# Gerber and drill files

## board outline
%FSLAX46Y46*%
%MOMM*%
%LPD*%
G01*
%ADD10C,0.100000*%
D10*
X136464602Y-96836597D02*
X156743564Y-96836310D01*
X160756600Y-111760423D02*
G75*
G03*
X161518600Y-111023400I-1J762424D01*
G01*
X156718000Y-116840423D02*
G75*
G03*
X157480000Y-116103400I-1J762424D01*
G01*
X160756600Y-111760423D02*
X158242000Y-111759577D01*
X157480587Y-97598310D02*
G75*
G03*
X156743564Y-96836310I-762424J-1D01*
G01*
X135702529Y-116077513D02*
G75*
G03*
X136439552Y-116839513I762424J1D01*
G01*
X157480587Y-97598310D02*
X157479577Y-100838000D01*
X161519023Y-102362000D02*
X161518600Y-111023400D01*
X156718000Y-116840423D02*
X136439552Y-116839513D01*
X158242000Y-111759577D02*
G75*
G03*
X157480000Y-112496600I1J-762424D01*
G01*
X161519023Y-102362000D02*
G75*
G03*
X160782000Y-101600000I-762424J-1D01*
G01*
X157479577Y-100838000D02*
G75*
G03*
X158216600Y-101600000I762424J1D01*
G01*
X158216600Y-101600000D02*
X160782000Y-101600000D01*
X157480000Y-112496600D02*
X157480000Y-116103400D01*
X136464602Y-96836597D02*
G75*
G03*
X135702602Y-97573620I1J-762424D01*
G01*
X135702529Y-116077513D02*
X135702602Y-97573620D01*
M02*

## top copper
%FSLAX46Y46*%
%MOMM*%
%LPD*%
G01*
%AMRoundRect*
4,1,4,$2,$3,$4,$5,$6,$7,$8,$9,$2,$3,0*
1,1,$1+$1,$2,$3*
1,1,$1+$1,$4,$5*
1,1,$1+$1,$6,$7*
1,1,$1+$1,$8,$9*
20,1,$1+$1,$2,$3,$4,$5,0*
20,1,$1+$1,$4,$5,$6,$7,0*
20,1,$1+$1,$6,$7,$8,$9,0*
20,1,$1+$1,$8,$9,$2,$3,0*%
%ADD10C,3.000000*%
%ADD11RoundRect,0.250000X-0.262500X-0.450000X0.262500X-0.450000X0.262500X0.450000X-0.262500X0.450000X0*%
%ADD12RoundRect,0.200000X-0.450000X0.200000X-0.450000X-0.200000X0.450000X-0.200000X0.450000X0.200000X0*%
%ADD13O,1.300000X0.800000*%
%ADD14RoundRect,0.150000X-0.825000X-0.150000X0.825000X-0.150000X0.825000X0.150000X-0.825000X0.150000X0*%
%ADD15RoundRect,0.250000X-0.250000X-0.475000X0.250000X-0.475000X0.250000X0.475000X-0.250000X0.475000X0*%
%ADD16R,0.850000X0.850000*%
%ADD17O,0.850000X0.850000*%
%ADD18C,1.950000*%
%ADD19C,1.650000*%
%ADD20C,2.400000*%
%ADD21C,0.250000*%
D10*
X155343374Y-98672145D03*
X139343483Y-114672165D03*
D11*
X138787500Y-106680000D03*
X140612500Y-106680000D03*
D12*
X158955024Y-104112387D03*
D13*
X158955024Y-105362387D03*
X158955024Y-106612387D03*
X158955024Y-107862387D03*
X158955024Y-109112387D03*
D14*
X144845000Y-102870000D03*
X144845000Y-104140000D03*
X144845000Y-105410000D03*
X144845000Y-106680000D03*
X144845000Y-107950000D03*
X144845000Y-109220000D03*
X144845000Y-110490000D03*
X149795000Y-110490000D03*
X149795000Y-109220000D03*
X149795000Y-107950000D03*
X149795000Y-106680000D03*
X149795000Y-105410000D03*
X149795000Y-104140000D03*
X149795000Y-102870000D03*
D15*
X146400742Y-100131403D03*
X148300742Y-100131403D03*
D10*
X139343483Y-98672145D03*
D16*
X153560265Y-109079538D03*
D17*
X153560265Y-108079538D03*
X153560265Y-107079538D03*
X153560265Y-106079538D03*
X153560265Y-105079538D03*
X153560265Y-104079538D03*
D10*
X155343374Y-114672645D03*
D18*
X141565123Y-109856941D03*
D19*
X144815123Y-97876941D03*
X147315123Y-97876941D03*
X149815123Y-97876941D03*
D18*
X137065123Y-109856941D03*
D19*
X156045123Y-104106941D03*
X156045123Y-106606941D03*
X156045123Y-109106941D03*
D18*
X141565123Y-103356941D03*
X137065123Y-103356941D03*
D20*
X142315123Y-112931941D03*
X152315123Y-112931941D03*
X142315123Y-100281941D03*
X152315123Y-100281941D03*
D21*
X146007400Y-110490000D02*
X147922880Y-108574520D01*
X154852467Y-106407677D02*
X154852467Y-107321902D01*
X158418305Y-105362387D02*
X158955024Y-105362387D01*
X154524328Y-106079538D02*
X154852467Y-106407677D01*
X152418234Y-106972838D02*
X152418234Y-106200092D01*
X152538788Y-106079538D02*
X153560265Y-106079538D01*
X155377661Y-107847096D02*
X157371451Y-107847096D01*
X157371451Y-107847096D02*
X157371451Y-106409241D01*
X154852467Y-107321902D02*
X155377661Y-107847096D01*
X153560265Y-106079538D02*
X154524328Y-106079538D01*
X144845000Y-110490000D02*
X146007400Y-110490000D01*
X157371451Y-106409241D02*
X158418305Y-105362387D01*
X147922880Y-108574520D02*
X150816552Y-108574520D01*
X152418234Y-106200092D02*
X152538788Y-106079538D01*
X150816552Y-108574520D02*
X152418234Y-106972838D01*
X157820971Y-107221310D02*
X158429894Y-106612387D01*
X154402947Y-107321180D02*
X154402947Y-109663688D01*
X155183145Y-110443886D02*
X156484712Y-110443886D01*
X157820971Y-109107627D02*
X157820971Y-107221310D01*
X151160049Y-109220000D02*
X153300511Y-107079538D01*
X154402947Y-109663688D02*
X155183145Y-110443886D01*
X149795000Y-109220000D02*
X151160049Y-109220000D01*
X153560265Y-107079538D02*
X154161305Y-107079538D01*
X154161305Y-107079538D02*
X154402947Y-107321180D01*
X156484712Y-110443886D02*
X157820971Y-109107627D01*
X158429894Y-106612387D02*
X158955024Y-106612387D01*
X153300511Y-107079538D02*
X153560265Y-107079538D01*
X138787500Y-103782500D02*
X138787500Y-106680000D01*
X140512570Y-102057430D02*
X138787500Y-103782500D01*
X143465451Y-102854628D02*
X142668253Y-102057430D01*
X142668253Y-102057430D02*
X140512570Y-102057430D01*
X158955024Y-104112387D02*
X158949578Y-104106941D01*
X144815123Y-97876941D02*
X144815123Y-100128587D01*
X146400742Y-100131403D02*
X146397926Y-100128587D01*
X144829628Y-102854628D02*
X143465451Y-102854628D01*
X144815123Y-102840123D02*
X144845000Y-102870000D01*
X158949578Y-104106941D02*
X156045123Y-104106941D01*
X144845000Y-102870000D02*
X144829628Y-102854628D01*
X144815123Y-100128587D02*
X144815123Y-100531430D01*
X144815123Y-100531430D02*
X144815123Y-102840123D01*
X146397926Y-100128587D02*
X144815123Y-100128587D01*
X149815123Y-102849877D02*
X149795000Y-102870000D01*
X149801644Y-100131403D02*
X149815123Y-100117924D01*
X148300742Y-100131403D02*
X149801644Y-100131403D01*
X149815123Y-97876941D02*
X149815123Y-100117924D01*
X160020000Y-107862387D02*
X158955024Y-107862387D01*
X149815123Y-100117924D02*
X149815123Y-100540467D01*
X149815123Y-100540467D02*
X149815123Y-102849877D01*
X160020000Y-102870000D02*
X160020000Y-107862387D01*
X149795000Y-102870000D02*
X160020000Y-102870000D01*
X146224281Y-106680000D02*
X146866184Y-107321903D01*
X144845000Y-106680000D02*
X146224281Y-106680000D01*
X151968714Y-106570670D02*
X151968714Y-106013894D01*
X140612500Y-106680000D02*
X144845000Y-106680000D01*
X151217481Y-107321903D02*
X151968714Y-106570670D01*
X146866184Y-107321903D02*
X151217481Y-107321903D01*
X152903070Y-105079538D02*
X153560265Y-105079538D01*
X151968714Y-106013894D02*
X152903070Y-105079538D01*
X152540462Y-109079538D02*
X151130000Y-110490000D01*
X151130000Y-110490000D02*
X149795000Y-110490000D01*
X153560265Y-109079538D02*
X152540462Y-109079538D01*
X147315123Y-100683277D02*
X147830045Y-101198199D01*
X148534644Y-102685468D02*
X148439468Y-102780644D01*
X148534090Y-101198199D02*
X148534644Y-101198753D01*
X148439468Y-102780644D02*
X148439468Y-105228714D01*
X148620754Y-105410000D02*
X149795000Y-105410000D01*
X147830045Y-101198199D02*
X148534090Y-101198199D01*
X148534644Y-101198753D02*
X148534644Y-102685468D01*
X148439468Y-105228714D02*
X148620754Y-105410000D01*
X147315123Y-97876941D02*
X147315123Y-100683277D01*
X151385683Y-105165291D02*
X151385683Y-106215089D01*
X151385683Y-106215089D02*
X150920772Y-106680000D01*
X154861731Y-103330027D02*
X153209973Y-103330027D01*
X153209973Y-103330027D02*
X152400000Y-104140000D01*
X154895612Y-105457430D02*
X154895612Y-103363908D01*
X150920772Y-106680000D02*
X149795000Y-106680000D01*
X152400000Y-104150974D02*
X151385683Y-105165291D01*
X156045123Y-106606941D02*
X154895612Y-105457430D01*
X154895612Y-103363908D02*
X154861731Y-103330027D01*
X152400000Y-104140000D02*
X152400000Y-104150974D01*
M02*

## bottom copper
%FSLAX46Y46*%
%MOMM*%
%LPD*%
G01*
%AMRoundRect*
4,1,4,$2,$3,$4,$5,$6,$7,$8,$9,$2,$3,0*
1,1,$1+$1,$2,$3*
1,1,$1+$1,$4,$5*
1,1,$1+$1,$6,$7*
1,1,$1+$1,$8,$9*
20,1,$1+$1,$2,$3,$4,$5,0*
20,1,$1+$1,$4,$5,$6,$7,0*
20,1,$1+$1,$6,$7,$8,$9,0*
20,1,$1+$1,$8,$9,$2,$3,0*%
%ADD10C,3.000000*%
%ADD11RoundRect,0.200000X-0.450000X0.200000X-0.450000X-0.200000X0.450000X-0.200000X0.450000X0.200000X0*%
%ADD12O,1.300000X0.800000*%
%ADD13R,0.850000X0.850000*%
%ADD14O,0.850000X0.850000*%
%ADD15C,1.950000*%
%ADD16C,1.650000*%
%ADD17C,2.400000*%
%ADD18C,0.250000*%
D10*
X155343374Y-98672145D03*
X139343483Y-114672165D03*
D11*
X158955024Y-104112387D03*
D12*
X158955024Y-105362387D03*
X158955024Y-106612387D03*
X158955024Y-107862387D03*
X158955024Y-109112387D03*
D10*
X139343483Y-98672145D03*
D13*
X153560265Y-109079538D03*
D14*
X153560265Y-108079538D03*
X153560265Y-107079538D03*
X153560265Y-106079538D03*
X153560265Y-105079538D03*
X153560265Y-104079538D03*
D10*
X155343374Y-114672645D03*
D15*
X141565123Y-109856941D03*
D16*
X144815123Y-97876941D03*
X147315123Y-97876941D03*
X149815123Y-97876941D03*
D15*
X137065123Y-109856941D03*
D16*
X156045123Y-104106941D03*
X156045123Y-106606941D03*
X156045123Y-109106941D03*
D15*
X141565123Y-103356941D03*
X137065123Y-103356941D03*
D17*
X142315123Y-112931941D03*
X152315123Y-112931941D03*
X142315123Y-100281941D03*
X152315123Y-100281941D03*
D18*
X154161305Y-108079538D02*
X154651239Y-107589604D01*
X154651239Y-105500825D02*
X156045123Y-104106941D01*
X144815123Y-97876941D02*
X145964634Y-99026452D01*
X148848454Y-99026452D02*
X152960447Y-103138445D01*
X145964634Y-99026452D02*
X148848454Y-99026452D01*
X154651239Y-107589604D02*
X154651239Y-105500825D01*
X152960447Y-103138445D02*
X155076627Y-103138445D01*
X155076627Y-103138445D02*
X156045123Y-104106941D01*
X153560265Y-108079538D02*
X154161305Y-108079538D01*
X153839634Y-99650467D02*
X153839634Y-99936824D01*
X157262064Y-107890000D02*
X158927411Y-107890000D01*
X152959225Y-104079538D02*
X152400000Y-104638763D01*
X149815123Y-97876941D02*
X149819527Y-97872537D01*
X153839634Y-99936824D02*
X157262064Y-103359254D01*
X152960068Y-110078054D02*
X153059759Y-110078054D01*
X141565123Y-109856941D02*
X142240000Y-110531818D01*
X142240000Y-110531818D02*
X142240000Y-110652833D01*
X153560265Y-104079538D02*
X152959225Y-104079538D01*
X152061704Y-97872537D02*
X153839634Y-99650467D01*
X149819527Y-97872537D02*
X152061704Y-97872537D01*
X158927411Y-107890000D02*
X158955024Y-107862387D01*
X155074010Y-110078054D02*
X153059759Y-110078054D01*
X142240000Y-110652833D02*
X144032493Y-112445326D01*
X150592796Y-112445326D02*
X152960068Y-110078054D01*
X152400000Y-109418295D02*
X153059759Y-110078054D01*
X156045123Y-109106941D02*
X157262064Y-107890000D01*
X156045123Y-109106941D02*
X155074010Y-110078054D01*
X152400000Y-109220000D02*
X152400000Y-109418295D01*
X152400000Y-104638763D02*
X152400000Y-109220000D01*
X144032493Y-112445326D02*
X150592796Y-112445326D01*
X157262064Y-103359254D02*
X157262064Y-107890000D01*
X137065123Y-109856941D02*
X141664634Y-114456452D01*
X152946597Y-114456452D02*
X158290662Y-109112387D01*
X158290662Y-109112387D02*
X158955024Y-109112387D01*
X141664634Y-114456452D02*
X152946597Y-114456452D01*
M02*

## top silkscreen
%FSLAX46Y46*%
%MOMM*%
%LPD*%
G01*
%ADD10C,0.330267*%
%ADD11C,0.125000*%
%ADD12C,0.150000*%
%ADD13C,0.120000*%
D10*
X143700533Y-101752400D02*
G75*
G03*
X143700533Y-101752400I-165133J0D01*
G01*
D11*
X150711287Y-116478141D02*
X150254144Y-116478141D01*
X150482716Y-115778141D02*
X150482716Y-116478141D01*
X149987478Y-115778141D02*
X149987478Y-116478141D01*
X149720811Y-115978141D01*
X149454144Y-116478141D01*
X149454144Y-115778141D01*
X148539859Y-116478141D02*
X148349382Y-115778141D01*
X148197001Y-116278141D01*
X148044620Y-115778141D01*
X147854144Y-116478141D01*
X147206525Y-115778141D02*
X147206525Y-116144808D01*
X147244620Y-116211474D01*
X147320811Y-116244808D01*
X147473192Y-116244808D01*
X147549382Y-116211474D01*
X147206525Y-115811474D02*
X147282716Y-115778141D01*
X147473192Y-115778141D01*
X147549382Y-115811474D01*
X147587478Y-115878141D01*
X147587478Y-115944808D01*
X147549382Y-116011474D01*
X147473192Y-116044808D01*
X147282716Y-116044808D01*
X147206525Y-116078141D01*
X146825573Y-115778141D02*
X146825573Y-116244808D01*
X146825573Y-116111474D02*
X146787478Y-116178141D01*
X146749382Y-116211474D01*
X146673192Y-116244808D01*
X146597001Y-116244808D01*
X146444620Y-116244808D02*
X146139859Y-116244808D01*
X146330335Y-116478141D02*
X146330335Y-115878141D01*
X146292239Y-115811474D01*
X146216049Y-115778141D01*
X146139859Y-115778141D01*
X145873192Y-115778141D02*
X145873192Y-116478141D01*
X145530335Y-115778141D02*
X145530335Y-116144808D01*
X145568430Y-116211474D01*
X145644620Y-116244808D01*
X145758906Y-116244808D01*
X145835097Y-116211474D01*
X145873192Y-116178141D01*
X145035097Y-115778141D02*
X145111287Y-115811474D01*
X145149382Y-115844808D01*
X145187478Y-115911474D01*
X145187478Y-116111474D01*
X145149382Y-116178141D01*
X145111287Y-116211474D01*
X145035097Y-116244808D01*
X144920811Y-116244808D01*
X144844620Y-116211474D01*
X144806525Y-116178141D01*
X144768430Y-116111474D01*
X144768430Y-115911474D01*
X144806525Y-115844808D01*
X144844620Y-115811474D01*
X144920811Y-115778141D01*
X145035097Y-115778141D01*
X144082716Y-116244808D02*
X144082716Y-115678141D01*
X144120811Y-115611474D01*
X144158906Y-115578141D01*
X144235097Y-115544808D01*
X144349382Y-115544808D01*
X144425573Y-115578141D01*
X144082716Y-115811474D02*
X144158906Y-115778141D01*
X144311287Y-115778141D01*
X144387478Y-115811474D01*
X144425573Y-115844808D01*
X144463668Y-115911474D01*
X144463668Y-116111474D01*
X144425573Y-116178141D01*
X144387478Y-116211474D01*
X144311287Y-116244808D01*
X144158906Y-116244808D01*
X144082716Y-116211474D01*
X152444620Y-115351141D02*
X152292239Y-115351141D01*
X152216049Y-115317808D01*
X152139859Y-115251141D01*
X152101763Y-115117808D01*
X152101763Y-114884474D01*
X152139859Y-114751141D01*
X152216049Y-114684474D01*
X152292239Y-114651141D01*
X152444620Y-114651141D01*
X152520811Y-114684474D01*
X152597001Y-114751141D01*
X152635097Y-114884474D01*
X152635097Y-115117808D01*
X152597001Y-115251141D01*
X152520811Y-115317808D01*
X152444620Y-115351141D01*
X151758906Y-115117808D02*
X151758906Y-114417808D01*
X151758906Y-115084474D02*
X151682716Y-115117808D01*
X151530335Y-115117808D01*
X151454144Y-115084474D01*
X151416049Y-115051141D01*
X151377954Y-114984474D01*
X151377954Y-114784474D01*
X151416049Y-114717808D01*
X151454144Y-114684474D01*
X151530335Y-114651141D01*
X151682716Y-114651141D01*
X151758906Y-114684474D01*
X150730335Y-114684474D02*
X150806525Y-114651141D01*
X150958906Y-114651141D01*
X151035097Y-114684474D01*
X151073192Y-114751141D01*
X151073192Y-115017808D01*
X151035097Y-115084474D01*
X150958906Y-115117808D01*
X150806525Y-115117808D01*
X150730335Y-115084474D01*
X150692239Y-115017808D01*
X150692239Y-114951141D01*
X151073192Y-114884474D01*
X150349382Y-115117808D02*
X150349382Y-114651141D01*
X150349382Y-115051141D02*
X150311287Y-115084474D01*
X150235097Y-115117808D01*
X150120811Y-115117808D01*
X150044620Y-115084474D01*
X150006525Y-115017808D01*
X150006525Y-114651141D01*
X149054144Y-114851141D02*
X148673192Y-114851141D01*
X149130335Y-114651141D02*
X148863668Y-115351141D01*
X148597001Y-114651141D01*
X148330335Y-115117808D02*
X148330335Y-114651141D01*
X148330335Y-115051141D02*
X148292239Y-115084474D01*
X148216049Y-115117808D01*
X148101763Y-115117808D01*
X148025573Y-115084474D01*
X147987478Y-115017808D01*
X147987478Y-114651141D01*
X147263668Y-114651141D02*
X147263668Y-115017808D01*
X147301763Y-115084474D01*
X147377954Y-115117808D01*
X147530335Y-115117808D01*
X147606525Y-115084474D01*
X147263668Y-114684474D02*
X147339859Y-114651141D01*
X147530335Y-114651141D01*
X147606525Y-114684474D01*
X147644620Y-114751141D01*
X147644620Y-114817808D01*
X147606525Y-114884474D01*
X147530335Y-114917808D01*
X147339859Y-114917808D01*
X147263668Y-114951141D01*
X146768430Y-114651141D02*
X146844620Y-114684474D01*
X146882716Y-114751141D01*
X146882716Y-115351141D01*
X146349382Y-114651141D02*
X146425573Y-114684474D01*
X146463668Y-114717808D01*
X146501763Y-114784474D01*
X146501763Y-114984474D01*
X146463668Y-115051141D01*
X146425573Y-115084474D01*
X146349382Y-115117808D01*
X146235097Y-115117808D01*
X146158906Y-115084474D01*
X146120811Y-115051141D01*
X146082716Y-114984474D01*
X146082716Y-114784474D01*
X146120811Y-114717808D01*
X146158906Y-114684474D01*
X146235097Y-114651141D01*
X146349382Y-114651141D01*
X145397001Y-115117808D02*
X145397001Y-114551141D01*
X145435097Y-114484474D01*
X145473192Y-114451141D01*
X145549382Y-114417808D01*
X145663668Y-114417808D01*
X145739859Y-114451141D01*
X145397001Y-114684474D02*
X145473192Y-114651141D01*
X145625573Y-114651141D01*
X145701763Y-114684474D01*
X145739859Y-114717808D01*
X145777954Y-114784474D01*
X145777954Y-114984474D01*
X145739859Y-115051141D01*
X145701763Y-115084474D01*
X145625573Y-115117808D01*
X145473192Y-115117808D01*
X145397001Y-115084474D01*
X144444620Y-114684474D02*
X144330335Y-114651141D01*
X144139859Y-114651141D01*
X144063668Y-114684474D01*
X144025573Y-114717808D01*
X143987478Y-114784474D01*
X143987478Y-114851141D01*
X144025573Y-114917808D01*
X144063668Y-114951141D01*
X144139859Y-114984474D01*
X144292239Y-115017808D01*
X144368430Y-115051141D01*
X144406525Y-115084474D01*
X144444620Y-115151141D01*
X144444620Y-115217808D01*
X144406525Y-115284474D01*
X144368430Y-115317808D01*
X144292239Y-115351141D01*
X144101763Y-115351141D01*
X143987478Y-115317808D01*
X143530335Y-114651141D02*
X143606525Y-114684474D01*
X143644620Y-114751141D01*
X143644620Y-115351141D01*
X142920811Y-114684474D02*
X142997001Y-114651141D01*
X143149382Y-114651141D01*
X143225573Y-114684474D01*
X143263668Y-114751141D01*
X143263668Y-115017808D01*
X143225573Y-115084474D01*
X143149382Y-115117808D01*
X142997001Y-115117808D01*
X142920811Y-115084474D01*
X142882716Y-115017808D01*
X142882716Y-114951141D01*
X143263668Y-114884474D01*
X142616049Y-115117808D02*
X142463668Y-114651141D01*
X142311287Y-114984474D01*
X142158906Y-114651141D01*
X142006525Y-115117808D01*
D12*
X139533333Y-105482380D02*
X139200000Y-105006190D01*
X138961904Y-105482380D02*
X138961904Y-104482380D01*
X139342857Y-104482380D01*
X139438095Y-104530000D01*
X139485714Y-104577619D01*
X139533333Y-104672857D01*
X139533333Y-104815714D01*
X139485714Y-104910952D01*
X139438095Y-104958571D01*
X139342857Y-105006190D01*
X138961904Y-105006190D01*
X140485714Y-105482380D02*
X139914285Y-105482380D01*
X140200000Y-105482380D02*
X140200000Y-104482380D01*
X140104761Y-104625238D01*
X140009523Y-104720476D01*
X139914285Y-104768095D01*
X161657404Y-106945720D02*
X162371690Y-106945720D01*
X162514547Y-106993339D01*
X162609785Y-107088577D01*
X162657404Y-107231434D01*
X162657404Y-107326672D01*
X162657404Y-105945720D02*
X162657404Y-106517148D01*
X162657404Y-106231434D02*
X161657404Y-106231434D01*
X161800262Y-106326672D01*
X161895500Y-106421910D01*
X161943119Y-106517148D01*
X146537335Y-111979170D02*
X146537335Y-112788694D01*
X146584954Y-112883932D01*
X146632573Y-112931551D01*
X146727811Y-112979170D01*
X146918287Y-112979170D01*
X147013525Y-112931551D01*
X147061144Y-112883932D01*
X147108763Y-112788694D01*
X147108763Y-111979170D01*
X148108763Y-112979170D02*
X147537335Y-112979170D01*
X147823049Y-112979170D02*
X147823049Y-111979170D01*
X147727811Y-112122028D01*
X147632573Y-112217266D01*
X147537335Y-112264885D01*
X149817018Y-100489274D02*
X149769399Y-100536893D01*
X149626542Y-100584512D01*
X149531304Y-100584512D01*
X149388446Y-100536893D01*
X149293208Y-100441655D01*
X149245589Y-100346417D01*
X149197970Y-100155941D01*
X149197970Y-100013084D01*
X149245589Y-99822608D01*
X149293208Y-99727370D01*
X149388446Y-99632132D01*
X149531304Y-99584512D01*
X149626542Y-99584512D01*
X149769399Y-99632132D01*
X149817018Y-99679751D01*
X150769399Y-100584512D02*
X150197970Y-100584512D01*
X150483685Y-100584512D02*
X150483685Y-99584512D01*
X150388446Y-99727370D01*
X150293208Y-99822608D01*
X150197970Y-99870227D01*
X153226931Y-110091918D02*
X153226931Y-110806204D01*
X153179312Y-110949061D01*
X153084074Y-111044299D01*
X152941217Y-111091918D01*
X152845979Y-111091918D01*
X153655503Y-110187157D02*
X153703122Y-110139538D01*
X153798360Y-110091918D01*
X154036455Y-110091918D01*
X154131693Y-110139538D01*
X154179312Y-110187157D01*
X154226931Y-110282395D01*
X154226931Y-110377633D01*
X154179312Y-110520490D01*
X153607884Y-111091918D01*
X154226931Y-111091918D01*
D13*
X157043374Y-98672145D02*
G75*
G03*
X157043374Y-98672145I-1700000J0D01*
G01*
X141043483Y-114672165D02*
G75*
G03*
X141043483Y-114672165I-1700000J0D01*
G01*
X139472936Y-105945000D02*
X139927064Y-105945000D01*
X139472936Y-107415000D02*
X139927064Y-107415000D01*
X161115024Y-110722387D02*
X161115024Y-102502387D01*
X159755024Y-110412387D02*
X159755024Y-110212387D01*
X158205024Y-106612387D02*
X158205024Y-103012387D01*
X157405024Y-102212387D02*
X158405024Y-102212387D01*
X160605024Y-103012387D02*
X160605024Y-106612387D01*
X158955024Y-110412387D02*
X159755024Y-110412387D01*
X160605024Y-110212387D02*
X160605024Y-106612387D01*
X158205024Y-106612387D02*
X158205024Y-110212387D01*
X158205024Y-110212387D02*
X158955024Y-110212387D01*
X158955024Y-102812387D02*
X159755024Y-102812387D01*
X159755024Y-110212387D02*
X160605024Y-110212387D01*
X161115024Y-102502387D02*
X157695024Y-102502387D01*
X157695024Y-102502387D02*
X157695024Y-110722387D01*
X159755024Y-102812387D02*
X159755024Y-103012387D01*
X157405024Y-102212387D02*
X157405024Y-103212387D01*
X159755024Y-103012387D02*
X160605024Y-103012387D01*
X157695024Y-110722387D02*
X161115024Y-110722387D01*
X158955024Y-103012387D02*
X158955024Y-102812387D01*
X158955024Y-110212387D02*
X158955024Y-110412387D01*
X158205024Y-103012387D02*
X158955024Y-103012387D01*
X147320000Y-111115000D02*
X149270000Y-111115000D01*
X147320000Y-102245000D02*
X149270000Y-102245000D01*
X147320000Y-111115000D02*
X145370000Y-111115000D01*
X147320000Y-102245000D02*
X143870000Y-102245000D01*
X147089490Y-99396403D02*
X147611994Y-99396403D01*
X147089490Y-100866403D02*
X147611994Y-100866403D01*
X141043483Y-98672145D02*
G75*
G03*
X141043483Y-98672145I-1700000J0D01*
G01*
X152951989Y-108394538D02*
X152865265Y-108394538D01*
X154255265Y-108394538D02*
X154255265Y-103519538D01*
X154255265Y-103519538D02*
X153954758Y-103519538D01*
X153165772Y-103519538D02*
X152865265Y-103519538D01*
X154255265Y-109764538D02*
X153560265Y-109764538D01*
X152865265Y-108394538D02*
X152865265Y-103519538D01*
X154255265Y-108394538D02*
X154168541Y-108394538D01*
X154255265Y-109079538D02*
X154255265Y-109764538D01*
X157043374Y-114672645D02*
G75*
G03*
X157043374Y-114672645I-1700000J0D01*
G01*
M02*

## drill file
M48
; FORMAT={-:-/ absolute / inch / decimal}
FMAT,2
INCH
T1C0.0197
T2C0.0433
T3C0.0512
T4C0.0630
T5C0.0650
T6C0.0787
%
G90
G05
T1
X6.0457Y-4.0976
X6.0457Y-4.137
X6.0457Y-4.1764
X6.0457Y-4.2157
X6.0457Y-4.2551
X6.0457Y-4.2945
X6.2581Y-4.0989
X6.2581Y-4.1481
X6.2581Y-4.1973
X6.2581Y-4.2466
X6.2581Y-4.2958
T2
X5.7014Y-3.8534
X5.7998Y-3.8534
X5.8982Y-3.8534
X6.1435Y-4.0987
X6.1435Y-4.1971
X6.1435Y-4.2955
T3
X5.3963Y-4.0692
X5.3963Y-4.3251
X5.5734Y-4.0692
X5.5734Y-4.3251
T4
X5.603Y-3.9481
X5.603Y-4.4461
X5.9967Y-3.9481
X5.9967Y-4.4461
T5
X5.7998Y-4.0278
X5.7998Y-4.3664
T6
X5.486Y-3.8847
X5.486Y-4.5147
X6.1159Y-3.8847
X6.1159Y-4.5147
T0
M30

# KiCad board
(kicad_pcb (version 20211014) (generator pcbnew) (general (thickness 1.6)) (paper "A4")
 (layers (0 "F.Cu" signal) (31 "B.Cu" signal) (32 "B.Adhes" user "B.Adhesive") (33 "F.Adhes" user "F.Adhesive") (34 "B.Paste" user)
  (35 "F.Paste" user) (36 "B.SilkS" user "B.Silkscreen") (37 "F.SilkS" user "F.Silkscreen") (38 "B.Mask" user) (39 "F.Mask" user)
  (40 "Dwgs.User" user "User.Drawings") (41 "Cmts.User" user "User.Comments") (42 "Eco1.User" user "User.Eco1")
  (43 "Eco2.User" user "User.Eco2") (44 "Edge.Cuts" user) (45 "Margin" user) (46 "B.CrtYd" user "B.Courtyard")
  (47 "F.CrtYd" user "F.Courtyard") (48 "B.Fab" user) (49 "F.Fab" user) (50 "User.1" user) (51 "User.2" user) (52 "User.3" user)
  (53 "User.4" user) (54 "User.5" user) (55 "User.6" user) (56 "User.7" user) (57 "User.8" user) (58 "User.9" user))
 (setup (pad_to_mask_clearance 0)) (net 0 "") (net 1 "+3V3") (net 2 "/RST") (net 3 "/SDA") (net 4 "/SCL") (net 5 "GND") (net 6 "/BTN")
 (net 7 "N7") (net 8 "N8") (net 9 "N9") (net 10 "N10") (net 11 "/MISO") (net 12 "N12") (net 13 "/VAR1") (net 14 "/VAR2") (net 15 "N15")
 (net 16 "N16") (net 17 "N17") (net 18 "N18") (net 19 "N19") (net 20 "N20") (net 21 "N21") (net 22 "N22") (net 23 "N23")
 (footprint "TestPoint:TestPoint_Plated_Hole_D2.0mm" (layer "F.Cu") (at 155.343374 98.672145) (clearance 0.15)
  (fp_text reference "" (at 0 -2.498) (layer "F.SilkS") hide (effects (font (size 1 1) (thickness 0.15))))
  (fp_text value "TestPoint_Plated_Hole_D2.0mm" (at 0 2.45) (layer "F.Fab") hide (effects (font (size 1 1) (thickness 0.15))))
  (fp_circle (center 0 0) (end 0 -1.7) (layer "F.SilkS") (width 0.12) (fill none))
  (pad "" thru_hole circle locked (at 0 0) (size 3 3) (drill 2) (layers *.Cu *.Mask)))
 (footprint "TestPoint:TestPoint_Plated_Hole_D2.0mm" (layer "F.Cu") (at 139.343483 114.672165) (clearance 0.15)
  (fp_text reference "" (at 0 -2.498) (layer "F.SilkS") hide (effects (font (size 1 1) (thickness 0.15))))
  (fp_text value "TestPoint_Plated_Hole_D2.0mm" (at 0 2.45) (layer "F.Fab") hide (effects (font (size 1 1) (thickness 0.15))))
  (fp_circle (center 0 0) (end 0 -1.7) (layer "F.SilkS") (width 0.12) (fill none))
  (pad "" thru_hole circle locked (at 0 0) (size 3 3) (drill 2) (layers *.Cu *.Mask)))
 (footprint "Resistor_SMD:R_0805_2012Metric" (layer "F.Cu") (at 139.7 106.68)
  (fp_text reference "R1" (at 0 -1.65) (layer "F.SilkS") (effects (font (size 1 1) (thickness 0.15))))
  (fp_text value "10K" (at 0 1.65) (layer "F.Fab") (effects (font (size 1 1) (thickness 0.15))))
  (fp_line (start -0.227064 -0.735) (end 0.227064 -0.735) (layer "F.SilkS") (width 0.12))
  (fp_line (start -0.227064 0.735) (end 0.227064 0.735) (layer "F.SilkS") (width 0.12))
  (pad "1" smd roundrect locked (at -0.9125 0) (size 1.025 1.4) (layers "F.Cu" "F.Paste" "F.Mask") (roundrect_rratio 0.243902439)
   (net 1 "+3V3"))
  (pad "2" smd roundrect locked (at 0.9125 0) (size 1.025 1.4) (layers "F.Cu" "F.Paste" "F.Mask") (roundrect_rratio 0.243902439)
   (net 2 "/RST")))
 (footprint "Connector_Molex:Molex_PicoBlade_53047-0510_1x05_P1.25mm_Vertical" (layer "F.Cu") (at 158.955024 104.112387 -90)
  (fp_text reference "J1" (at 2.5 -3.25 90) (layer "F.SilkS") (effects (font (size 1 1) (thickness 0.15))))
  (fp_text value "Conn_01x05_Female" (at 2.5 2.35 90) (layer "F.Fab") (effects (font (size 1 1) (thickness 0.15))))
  (fp_line (start 6.61 -2.16) (end -1.61 -2.16) (layer "F.SilkS") (width 0.12))
  (fp_line (start 6.3 -0.8) (end 6.1 -0.8) (layer "F.SilkS") (width 0.12))
  (fp_line (start 2.5 0.75) (end -1.1 0.75) (layer "F.SilkS") (width 0.12))
  (fp_line (start -1.9 1.55) (end -1.9 0.55) (layer "F.SilkS") (width 0.12))
  (fp_line (start -1.1 -1.65) (end 2.5 -1.65) (layer "F.SilkS") (width 0.12))
  (fp_line (start 6.3 0) (end 6.3 -0.8) (layer "F.SilkS") (width 0.12))
  (fp_line (start 6.1 -1.65) (end 2.5 -1.65) (layer "F.SilkS") (width 0.12))
  (fp_line (start 2.5 0.75) (end 6.1 0.75) (layer "F.SilkS") (width 0.12))
  (fp_line (start 6.1 0.75) (end 6.1 0) (layer "F.SilkS") (width 0.12))
  (fp_line (start -1.3 0) (end -1.3 -0.8) (layer "F.SilkS") (width 0.12))
  (fp_line (start 6.1 -0.8) (end 6.1 -1.65) (layer "F.SilkS") (width 0.12))
  (fp_line (start -1.61 -2.16) (end -1.61 1.26) (layer "F.SilkS") (width 0.12))
  (fp_line (start -1.61 1.26) (end 6.61 1.26) (layer "F.SilkS") (width 0.12))
  (fp_line (start -1.3 -0.8) (end -1.1 -0.8) (layer "F.SilkS") (width 0.12))
  (fp_line (start -1.9 1.55) (end -0.9 1.55) (layer "F.SilkS") (width 0.12))
  (fp_line (start -1.1 -0.8) (end -1.1 -1.65) (layer "F.SilkS") (width 0.12))
  (fp_line (start 6.61 1.26) (end 6.61 -2.16) (layer "F.SilkS") (width 0.12))
  (fp_line (start -1.1 0) (end -1.3 0) (layer "F.SilkS") (width 0.12))
  (fp_line (start 6.1 0) (end 6.3 0) (layer "F.SilkS") (width 0.12))
  (fp_line (start -1.1 0.75) (end -1.1 0) (layer "F.SilkS") (width 0.12))
  (pad "1" thru_hole roundrect locked (at 0 0 270) (size 0.8 1.3) (drill 0.5) (layers *.Cu *.Mask) (roundrect_rratio 0.25) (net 1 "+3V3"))
  (pad "2" thru_hole oval locked (at 1.25 0 270) (size 0.8 1.3) (drill 0.5) (layers *.Cu *.Mask) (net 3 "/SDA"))
  (pad "3" thru_hole oval locked (at 2.5 0 270) (size 0.8 1.3) (drill 0.5) (layers *.Cu *.Mask) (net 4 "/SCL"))
  (pad "4" thru_hole oval locked (at 3.75 0 270) (size 0.8 1.3) (drill 0.5) (layers *.Cu *.Mask) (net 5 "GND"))
  (pad "5" thru_hole oval locked (at 5 0 270) (size 0.8 1.3) (drill 0.5) (layers *.Cu *.Mask) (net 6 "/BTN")))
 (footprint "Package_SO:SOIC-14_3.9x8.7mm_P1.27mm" (layer "F.Cu") (at 147.32 106.68) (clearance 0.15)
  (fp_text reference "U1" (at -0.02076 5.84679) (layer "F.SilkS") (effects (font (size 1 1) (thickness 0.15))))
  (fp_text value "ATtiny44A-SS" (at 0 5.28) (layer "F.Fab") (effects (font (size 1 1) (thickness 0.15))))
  (fp_line (start 0 4.435) (end 1.95 4.435) (layer "F.SilkS") (width 0.12))
  (fp_line (start 0 -4.435) (end 1.95 -4.435) (layer "F.SilkS") (width 0.12))
  (fp_line (start 0 4.435) (end -1.95 4.435) (layer "F.SilkS") (width 0.12))
  (fp_line (start 0 -4.435) (end -3.45 -4.435) (layer "F.SilkS") (width 0.12))
  (pad "1" smd roundrect locked (at -2.475 -3.81) (size 1.95 0.6) (layers "F.Cu" "F.Paste" "F.Mask") (roundrect_rratio 0.25) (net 1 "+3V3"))
  (pad "2" smd roundrect locked (at -2.475 -2.54) (size 1.95 0.6) (layers "F.Cu" "F.Paste" "F.Mask") (roundrect_rratio 0.25) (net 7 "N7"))
  (pad "3" smd roundrect locked (at -2.475 -1.27) (size 1.95 0.6) (layers "F.Cu" "F.Paste" "F.Mask") (roundrect_rratio 0.25) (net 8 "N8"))
  (pad "4" smd roundrect locked (at -2.475 0) (size 1.95 0.6) (layers "F.Cu" "F.Paste" "F.Mask") (roundrect_rratio 0.25) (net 2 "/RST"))
  (pad "5" smd roundrect locked (at -2.475 1.27) (size 1.95 0.6) (layers "F.Cu" "F.Paste" "F.Mask") (roundrect_rratio 0.25) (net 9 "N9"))
  (pad "6" smd roundrect locked (at -2.475 2.54) (size 1.95 0.6) (layers "F.Cu" "F.Paste" "F.Mask") (roundrect_rratio 0.25) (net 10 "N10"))
  (pad "7" smd roundrect locked (at -2.475 3.81) (size 1.95 0.6) (layers "F.Cu" "F.Paste" "F.Mask") (roundrect_rratio 0.25) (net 3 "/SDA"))
  (pad "8" smd roundrect locked (at 2.475 3.81) (size 1.95 0.6) (layers "F.Cu" "F.Paste" "F.Mask") (roundrect_rratio 0.25) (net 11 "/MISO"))
  (pad "9" smd roundrect locked (at 2.475 2.54) (size 1.95 0.6) (layers "F.Cu" "F.Paste" "F.Mask") (roundrect_rratio 0.25) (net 4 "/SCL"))
  (pad "10" smd roundrect locked (at 2.475 1.27) (size 1.95 0.6) (layers "F.Cu" "F.Paste" "F.Mask") (roundrect_rratio 0.25) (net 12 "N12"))
  (pad "11" smd roundrect locked (at 2.475 0) (size 1.95 0.6) (layers "F.Cu" "F.Paste" "F.Mask") (roundrect_rratio 0.25) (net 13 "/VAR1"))
  (pad "12" smd roundrect locked (at 2.475 -1.27) (size 1.95 0.6) (layers "F.Cu" "F.Paste" "F.Mask") (roundrect_rratio 0.25)
   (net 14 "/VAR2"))
  (pad "13" smd roundrect locked (at 2.475 -2.54) (size 1.95 0.6) (layers "F.Cu" "F.Paste" "F.Mask") (roundrect_rratio 0.25) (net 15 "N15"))
  (pad "14" smd roundrect locked (at 2.475 -3.81) (size 1.95 0.6) (layers "F.Cu" "F.Paste" "F.Mask") (roundrect_rratio 0.25) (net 5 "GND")))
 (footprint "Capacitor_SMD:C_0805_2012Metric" (layer "F.Cu") (at 147.350742 100.131403)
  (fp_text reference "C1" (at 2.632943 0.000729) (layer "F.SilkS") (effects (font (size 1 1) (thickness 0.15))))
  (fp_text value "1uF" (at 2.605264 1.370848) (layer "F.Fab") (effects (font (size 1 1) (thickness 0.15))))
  (fp_line (start -0.261252 -0.735) (end 0.261252 -0.735) (layer "F.SilkS") (width 0.12))
  (fp_line (start -0.261252 0.735) (end 0.261252 0.735) (layer "F.SilkS") (width 0.12))
  (pad "1" smd roundrect locked (at -0.95 0) (size 1 1.45) (layers "F.Cu" "F.Paste" "F.Mask") (roundrect_rratio 0.25) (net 1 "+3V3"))
  (pad "2" smd roundrect locked (at 0.95 0) (size 1 1.45) (layers "F.Cu" "F.Paste" "F.Mask") (roundrect_rratio 0.25) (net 5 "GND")))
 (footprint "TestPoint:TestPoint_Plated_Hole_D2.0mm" (layer "F.Cu") (at 139.343483 98.672145)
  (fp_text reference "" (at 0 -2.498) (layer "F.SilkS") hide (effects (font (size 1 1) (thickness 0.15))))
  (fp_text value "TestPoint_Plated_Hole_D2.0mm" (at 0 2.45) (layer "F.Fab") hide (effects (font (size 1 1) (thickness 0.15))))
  (fp_circle (center 0 0) (end 0 -1.7) (layer "F.SilkS") (width 0.12) (fill none))
  (pad "" thru_hole circle locked (at 0 0) (size 3 3) (drill 2) (layers *.Cu *.Mask)))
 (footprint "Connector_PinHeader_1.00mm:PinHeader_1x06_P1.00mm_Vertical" (layer "F.Cu") (at 153.560265 109.079538 180) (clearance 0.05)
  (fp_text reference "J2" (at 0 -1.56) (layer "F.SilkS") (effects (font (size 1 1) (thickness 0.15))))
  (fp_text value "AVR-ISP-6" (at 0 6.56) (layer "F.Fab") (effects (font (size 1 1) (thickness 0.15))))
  (fp_line (start 0.608276 0.685) (end 0.695 0.685) (layer "F.SilkS") (width 0.12))
  (fp_line (start -0.695 0.685) (end -0.695 5.56) (layer "F.SilkS") (width 0.12))
  (fp_line (start -0.695 5.56) (end -0.394493 5.56) (layer "F.SilkS") (width 0.12))
  (fp_line (start 0.394493 5.56) (end 0.695 5.56) (layer "F.SilkS") (width 0.12))
  (fp_line (start -0.695 -0.685) (end 0 -0.685) (layer "F.SilkS") (width 0.12))
  (fp_line (start 0.695 0.685) (end 0.695 5.56) (layer "F.SilkS") (width 0.12))
  (fp_line (start -0.695 0.685) (end -0.608276 0.685) (layer "F.SilkS") (width 0.12))
  (fp_line (start -0.695 0) (end -0.695 -0.685) (layer "F.SilkS") (width 0.12))
  (pad "1" thru_hole rect locked (at 0 0 180) (size 0.85 0.85) (drill 0.5) (layers *.Cu *.Mask) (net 11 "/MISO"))
  (pad "2" thru_hole oval locked (at 0 1 180) (size 0.85 0.85) (drill 0.5) (layers *.Cu *.Mask) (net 1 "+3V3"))
  (pad "3" thru_hole oval locked (at 0 2 180) (size 0.85 0.85) (drill 0.5) (layers *.Cu *.Mask) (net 4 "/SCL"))
  (pad "4" thru_hole oval locked (at 0 3 180) (size 0.85 0.85) (drill 0.5) (layers *.Cu *.Mask) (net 3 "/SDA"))
  (pad "5" thru_hole oval locked (at 0 4 180) (size 0.85 0.85) (drill 0.5) (layers *.Cu *.Mask) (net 2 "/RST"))
  (pad "6" thru_hole oval locked (at 0 5 180) (size 0.85 0.85) (drill 0.5) (layers *.Cu *.Mask) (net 5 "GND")))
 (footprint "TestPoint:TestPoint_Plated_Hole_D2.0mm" (layer "F.Cu") (at 155.343374 114.672645)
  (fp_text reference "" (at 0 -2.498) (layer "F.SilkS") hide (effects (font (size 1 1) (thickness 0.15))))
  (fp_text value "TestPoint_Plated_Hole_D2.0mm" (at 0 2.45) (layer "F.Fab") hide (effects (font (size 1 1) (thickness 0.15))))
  (fp_circle (center 0 0) (end 0 -1.7) (layer "F.SilkS") (width 0.12) (fill none))
  (pad "" thru_hole circle locked (at 0 0) (size 3 3) (drill 2) (layers *.Cu *.Mask)))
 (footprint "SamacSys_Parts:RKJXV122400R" (layer "B.Cu") (at 144.815123 97.876941 90)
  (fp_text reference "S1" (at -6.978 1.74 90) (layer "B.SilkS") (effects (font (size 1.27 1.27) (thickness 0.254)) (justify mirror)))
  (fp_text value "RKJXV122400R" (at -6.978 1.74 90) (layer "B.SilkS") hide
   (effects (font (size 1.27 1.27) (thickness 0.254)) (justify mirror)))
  (pad "A1" thru_hole circle locked (at -11.98 -3.25 90) (size 1.95 1.95) (drill 1.3) (layers *.Cu *.Mask) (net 5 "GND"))
  (pad "A11" thru_hole circle locked (at 0 0 90) (size 1.65 1.65) (drill 1.1) (layers *.Cu *.Mask) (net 1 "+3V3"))
  (pad "A12" thru_hole circle locked (at 0 2.5 90) (size 1.65 1.65) (drill 1.1) (layers *.Cu *.Mask) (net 14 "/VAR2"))
  (pad "A13" thru_hole circle locked (at 0 5 90) (size 1.65 1.65) (drill 1.1) (layers *.Cu *.Mask) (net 5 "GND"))
  (pad "B1" thru_hole circle locked (at -11.98 -7.75 90) (size 1.95 1.95) (drill 1.3) (layers *.Cu *.Mask) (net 6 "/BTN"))
  (pad "B11" thru_hole circle locked (at -6.23 11.23 90) (size 1.65 1.65) (drill 1.1) (layers *.Cu *.Mask) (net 1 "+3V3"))
  (pad "B12" thru_hole circle locked (at -8.73 11.23 90) (size 1.65 1.65) (drill 1.1) (layers *.Cu *.Mask) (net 13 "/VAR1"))
  (pad "B13" thru_hole circle locked (at -11.23 11.23 90) (size 1.65 1.65) (drill 1.1) (layers *.Cu *.Mask) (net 5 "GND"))
  (pad "C1" thru_hole circle locked (at -5.48 -3.25 90) (size 1.95 1.95) (drill 1.3) (layers *.Cu *.Mask) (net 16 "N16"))
  (pad "D1" thru_hole circle locked (at -5.48 -7.75 90) (size 1.95 1.95) (drill 1.3) (layers *.Cu *.Mask) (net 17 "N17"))
  (pad "MH1" thru_hole circle locked (at -15.055 -2.5 90) (size 2.4 2.4) (drill 1.6) (layers *.Cu *.Mask) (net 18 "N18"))
  (pad "MH2" thru_hole circle locked (at -15.055 7.5 90) (size 2.4 2.4) (drill 1.6) (layers *.Cu *.Mask) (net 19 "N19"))
  (pad "MH3" thru_hole circle locked (at -2.405 -2.5 90) (size 2.4 2.4) (drill 1.6) (layers *.Cu *.Mask) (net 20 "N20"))
  (pad "MH4" thru_hole circle locked (at -2.405 7.5 90) (size 2.4 2.4) (drill 1.6) (layers *.Cu *.Mask) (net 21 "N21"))
  (pad "MH5" thru_hole circle locked (at -13.03 2.5 90) (size 0 0) (drill 1.65) (layers *.Cu *.Mask) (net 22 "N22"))
  (pad "MH6" thru_hole circle locked (at -4.43 2.5 90) (size 0 0) (drill 1.65) (layers *.Cu *.Mask) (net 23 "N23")))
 (gr_circle (center 143.5354 101.7524) (end 143.7894 101.7778) (layer "F.SilkS") (width 0.15) (fill solid))
 (gr_line (start 136.464602 96.836597) (end 156.743564 96.83631) (layer "Edge.Cuts") (width 0.1))
 (gr_arc (start 161.5186 111.0234) (mid 161.286658 111.546021) (end 160.7566 111.760423) (layer "Edge.Cuts") (width 0.1))
 (gr_arc (start 157.48 116.1034) (mid 157.248058 116.626021) (end 156.718 116.840423) (layer "Edge.Cuts") (width 0.1))
 (gr_line (start 160.7566 111.760423) (end 158.242 111.759577) (layer "Edge.Cuts") (width 0.1))
 (gr_arc (start 156.743564 96.83631) (mid 157.266185 97.068252) (end 157.480587 97.59831) (layer "Edge.Cuts") (width 0.1))
 (gr_arc (start 136.439552 116.839513) (mid 135.916931 116.607571) (end 135.702529 116.077513) (layer "Edge.Cuts") (width 0.1))
 (gr_line (start 157.480587 97.59831) (end 157.479577 100.838) (layer "Edge.Cuts") (width 0.1))
 (gr_line (start 161.519023 102.362) (end 161.5186 111.0234) (layer "Edge.Cuts") (width 0.1))
 (gr_line (start 156.718 116.840423) (end 136.439552 116.839513) (layer "Edge.Cuts") (width 0.1))
 (gr_arc (start 157.48 112.4966) (mid 157.711942 111.973979) (end 158.242 111.759577) (layer "Edge.Cuts") (width 0.1))
 (gr_arc (start 160.782 101.6) (mid 161.304621 101.831942) (end 161.519023 102.362) (layer "Edge.Cuts") (width 0.1))
 (gr_arc (start 158.2166 101.6) (mid 157.693979 101.368058) (end 157.479577 100.838) (layer "Edge.Cuts") (width 0.1))
 (gr_line (start 158.2166 101.6) (end 160.782 101.6) (layer "Edge.Cuts") (width 0.1))
 (gr_line (start 157.48 112.4966) (end 157.48 116.1034) (layer "Edge.Cuts") (width 0.1))
 (gr_arc (start 135.702602 97.57362) (mid 135.934544 97.050999) (end 136.464602 96.836597) (layer "Edge.Cuts") (width 0.1))
 (gr_line (start 135.702529 116.077513) (end 135.702602 97.57362) (layer "Edge.Cuts") (width 0.1))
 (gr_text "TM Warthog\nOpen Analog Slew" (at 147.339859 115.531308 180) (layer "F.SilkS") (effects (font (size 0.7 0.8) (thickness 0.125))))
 (segment (start 146.0074 110.49) (end 147.92288 108.57452) (width 0.25) (layer "F.Cu") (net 3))
 (segment (start 154.852467 106.407677) (end 154.852467 107.321902) (width 0.25) (layer "F.Cu") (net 3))
 (segment (start 158.418305 105.362387) (end 158.955024 105.362387) (width 0.25) (layer "F.Cu") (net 3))
 (segment (start 154.524328 106.079538) (end 154.852467 106.407677) (width 0.25) (layer "F.Cu") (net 3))
 (segment (start 152.418234 106.972838) (end 152.418234 106.200092) (width 0.25) (layer "F.Cu") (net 3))
 (segment (start 152.538788 106.079538) (end 153.560265 106.079538) (width 0.25) (layer "F.Cu") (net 3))
 (segment (start 155.377661 107.847096) (end 157.371451 107.847096) (width 0.25) (layer "F.Cu") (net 3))
 (segment (start 157.371451 107.847096) (end 157.371451 106.409241) (width 0.25) (layer "F.Cu") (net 3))
 (segment (start 154.852467 107.321902) (end 155.377661 107.847096) (width 0.25) (layer "F.Cu") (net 3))
 (segment (start 153.560265 106.079538) (end 154.524328 106.079538) (width 0.25) (layer "F.Cu") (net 3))
 (segment (start 144.845 110.49) (end 146.0074 110.49) (width 0.25) (layer "F.Cu") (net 3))
 (segment (start 157.371451 106.409241) (end 158.418305 105.362387) (width 0.25) (layer "F.Cu") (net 3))
 (segment (start 147.92288 108.57452) (end 150.816552 108.57452) (width 0.25) (layer "F.Cu") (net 3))
 (segment (start 152.418234 106.200092) (end 152.538788 106.079538) (width 0.25) (layer "F.Cu") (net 3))
 (segment (start 150.816552 108.57452) (end 152.418234 106.972838) (width 0.25) (layer "F.Cu") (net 3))
 (segment (start 157.820971 107.22131) (end 158.429894 106.612387) (width 0.25) (layer "F.Cu") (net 4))
 (segment (start 154.402947 107.32118) (end 154.402947 109.663688) (width 0.25) (layer "F.Cu") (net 4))
 (segment (start 155.183145 110.443886) (end 156.484712 110.443886) (width 0.25) (layer "F.Cu") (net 4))
 (segment (start 157.820971 109.107627) (end 157.820971 107.22131) (width 0.25) (layer "F.Cu") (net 4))
 (segment (start 151.160049 109.22) (end 153.300511 107.079538) (width 0.25) (layer "F.Cu") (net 4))
 (segment (start 154.402947 109.663688) (end 155.183145 110.443886) (width 0.25) (layer "F.Cu") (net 4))
 (segment (start 149.795 109.22) (end 151.160049 109.22) (width 0.25) (layer "F.Cu") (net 4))
 (segment (start 153.560265 107.079538) (end 154.161305 107.079538) (width 0.25) (layer "F.Cu") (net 4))
 (segment (start 154.161305 107.079538) (end 154.402947 107.32118) (width 0.25) (layer "F.Cu") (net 4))
 (segment (start 156.484712 110.443886) (end 157.820971 109.107627) (width 0.25) (layer "F.Cu") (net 4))
 (segment (start 158.429894 106.612387) (end 158.955024 106.612387) (width 0.25) (layer "F.Cu") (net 4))
 (segment (start 153.300511 107.079538) (end 153.560265 107.079538) (width 0.25) (layer "F.Cu") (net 4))
 (segment (start 138.7875 103.7825) (end 138.7875 106.68) (width 0.25) (layer "F.Cu") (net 1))
 (segment (start 140.51257 102.05743) (end 138.7875 103.7825) (width 0.25) (layer "F.Cu") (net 1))
 (segment (start 143.465451 102.854628) (end 142.668253 102.05743) (width 0.25) (layer "F.Cu") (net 1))
 (segment (start 142.668253 102.05743) (end 140.51257 102.05743) (width 0.25) (layer "F.Cu") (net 1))
 (segment (start 158.955024 104.112387) (end 158.949578 104.106941) (width 0.25) (layer "F.Cu") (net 1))
 (segment (start 144.815123 97.876941) (end 144.815123 100.128587) (width 0.25) (layer "F.Cu") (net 1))
 (segment (start 146.400742 100.131403) (end 146.397926 100.128587) (width 0.25) (layer "F.Cu") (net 1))
 (segment (start 144.829628 102.854628) (end 143.465451 102.854628) (width 0.25) (layer "F.Cu") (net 1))
 (segment (start 144.815123 102.840123) (end 144.845 102.87) (width 0.25) (layer "F.Cu") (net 1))
 (segment (start 158.949578 104.106941) (end 156.045123 104.106941) (width 0.25) (layer "F.Cu") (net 1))
 (segment (start 144.845 102.87) (end 144.829628 102.854628) (width 0.25) (layer "F.Cu") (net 1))
 (segment (start 144.815123 100.128587) (end 144.815123 100.53143) (width 0.25) (layer "F.Cu") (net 1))
 (segment (start 144.815123 100.53143) (end 144.815123 102.840123) (width 0.25) (layer "F.Cu") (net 1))
 (segment (start 146.397926 100.128587) (end 144.815123 100.128587) (width 0.25) (layer "F.Cu") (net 1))
 (segment (start 154.161305 108.079538) (end 154.651239 107.589604) (width 0.25) (layer "B.Cu") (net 1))
 (segment (start 154.651239 105.500825) (end 156.045123 104.106941) (width 0.25) (layer "B.Cu") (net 1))
 (segment (start 144.815123 97.876941) (end 145.964634 99.026452) (width 0.25) (layer "B.Cu") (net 1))
 (segment (start 148.848454 99.026452) (end 152.960447 103.138445) (width 0.25) (layer "B.Cu") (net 1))
 (segment (start 145.964634 99.026452) (end 148.848454 99.026452) (width 0.25) (layer "B.Cu") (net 1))
 (segment (start 154.651239 107.589604) (end 154.651239 105.500825) (width 0.25) (layer "B.Cu") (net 1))
 (segment (start 152.960447 103.138445) (end 155.076627 103.138445) (width 0.25) (layer "B.Cu") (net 1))
 (segment (start 155.076627 103.138445) (end 156.045123 104.106941) (width 0.25) (layer "B.Cu") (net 1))
 (segment (start 153.560265 108.079538) (end 154.161305 108.079538) (width 0.25) (layer "B.Cu") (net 1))
 (segment (start 149.815123 102.849877) (end 149.795 102.87) (width 0.25) (layer "F.Cu") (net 5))
 (segment (start 149.801644 100.131403) (end 149.815123 100.117924) (width 0.25) (layer "F.Cu") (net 5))
 (segment (start 148.300742 100.131403) (end 149.801644 100.131403) (width 0.25) (layer "F.Cu") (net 5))
 (segment (start 149.815123 97.876941) (end 149.815123 100.117924) (width 0.25) (layer "F.Cu") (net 5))
 (segment (start 160.02 107.862387) (end 158.955024 107.862387) (width 0.25) (layer "F.Cu") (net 5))
 (segment (start 149.815123 100.117924) (end 149.815123 100.540467) (width 0.25) (layer "F.Cu") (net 5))
 (segment (start 149.815123 100.540467) (end 149.815123 102.849877) (width 0.25) (layer "F.Cu") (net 5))
 (segment (start 160.02 102.87) (end 160.02 107.862387) (width 0.25) (layer "F.Cu") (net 5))
 (segment (start 149.795 102.87) (end 160.02 102.87) (width 0.25) (layer "F.Cu") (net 5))
 (segment (start 153.839634 99.650467) (end 153.839634 99.936824) (width 0.25) (layer "B.Cu") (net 5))
 (segment (start 157.262064 107.89) (end 158.927411 107.89) (width 0.25) (layer "B.Cu") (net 5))
 (segment (start 152.959225 104.079538) (end 152.4 104.638763) (width 0.25) (layer "B.Cu") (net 5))
 (segment (start 149.815123 97.876941) (end 149.819527 97.872537) (width 0.25) (layer "B.Cu") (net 5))
 (segment (start 153.839634 99.936824) (end 157.262064 103.359254) (width 0.25) (layer "B.Cu") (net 5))
 (segment (start 152.960068 110.078054) (end 153.059759 110.078054) (width 0.25) (layer "B.Cu") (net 5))
 (segment (start 141.565123 109.856941) (end 142.24 110.531818) (width 0.25) (layer "B.Cu") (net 5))
 (segment (start 142.24 110.531818) (end 142.24 110.652833) (width 0.25) (layer "B.Cu") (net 5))
 (segment (start 153.560265 104.079538) (end 152.959225 104.079538) (width 0.25) (layer "B.Cu") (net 5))
 (segment (start 152.061704 97.872537) (end 153.839634 99.650467) (width 0.25) (layer "B.Cu") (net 5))
 (segment (start 149.819527 97.872537) (end 152.061704 97.872537) (width 0.25) (layer "B.Cu") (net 5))
 (segment (start 158.927411 107.89) (end 158.955024 107.862387) (width 0.25) (layer "B.Cu") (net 5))
 (segment (start 155.07401 110.078054) (end 153.059759 110.078054) (width 0.25) (layer "B.Cu") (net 5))
 (segment (start 142.24 110.652833) (end 144.032493 112.445326) (width 0.25) (layer "B.Cu") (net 5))
 (segment (start 150.592796 112.445326) (end 152.960068 110.078054) (width 0.25) (layer "B.Cu") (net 5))
 (segment (start 152.4 109.418295) (end 153.059759 110.078054) (width 0.25) (layer "B.Cu") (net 5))
 (segment (start 156.045123 109.106941) (end 157.262064 107.89) (width 0.25) (layer "B.Cu") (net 5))
 (segment (start 156.045123 109.106941) (end 155.07401 110.078054) (width 0.25) (layer "B.Cu") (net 5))
 (segment (start 152.4 109.22) (end 152.4 109.418295) (width 0.25) (layer "B.Cu") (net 5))
 (segment (start 152.4 104.638763) (end 152.4 109.22) (width 0.25) (layer "B.Cu") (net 5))
 (segment (start 144.032493 112.445326) (end 150.592796 112.445326) (width 0.25) (layer "B.Cu") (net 5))
 (segment (start 157.262064 103.359254) (end 157.262064 107.89) (width 0.25) (layer "B.Cu") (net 5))
 (segment (start 137.065123 109.856941) (end 141.664634 114.456452) (width 0.25) (layer "B.Cu") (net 6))
 (segment (start 152.946597 114.456452) (end 158.290662 109.112387) (width 0.25) (layer "B.Cu") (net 6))
 (segment (start 158.290662 109.112387) (end 158.955024 109.112387) (width 0.25) (layer "B.Cu") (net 6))
 (segment (start 141.664634 114.456452) (end 152.946597 114.456452) (width 0.25) (layer "B.Cu") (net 6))
 (segment (start 146.224281 106.68) (end 146.866184 107.321903) (width 0.25) (layer "F.Cu") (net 2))
 (segment (start 144.845 106.68) (end 146.224281 106.68) (width 0.25) (layer "F.Cu") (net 2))
 (segment (start 151.968714 106.57067) (end 151.968714 106.013894) (width 0.25) (layer "F.Cu") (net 2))
 (segment (start 140.6125 106.68) (end 144.845 106.68) (width 0.25) (layer "F.Cu") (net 2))
 (segment (start 151.217481 107.321903) (end 151.968714 106.57067) (width 0.25) (layer "F.Cu") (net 2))
 (segment (start 146.866184 107.321903) (end 151.217481 107.321903) (width 0.25) (layer "F.Cu") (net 2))
 (segment (start 152.90307 105.079538) (end 153.560265 105.079538) (width 0.25) (layer "F.Cu") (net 2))
 (segment (start 151.968714 106.013894) (end 152.90307 105.079538) (width 0.25) (layer "F.Cu") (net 2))
 (segment (start 152.540462 109.079538) (end 151.13 110.49) (width 0.25) (layer "F.Cu") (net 11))
 (segment (start 151.13 110.49) (end 149.795 110.49) (width 0.25) (layer "F.Cu") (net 11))
 (segment (start 153.560265 109.079538) (end 152.540462 109.079538) (width 0.25) (layer "F.Cu") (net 11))
 (segment (start 147.315123 100.683277) (end 147.830045 101.198199) (width 0.25) (layer "F.Cu") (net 14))
 (segment (start 148.534644 102.685468) (end 148.439468 102.780644) (width 0.25) (layer "F.Cu") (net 14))
 (segment (start 148.53409 101.198199) (end 148.534644 101.198753) (width 0.25) (layer "F.Cu") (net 14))
 (segment (start 148.439468 102.780644) (end 148.439468 105.228714) (width 0.25) (layer "F.Cu") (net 14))
 (segment (start 148.620754 105.41) (end 149.795 105.41) (width 0.25) (layer "F.Cu") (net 14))
 (segment (start 147.830045 101.198199) (end 148.53409 101.198199) (width 0.25) (layer "F.Cu") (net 14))
 (segment (start 148.534644 101.198753) (end 148.534644 102.685468) (width 0.25) (layer "F.Cu") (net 14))
 (segment (start 148.439468 105.228714) (end 148.620754 105.41) (width 0.25) (layer "F.Cu") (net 14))
 (segment (start 147.315123 97.876941) (end 147.315123 100.683277) (width 0.25) (layer "F.Cu") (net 14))
 (segment (start 151.385683 105.165291) (end 151.385683 106.215089) (width 0.25) (layer "F.Cu") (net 13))
 (segment (start 151.385683 106.215089) (end 150.920772 106.68) (width 0.25) (layer "F.Cu") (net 13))
 (segment (start 154.861731 103.330027) (end 153.209973 103.330027) (width 0.25) (layer "F.Cu") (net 13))
 (segment (start 153.209973 103.330027) (end 152.4 104.14) (width 0.25) (layer "F.Cu") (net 13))
 (segment (start 154.895612 105.45743) (end 154.895612 103.363908) (width 0.25) (layer "F.Cu") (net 13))
 (segment (start 150.920772 106.68) (end 149.795 106.68) (width 0.25) (layer "F.Cu") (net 13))
 (segment (start 152.4 104.150974) (end 151.385683 105.165291) (width 0.25) (layer "F.Cu") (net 13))
 (segment (start 156.045123 106.606941) (end 154.895612 105.45743) (width 0.25) (layer "F.Cu") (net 13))
 (segment (start 154.895612 103.363908) (end 154.861731 103.330027) (width 0.25) (layer "F.Cu") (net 13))
 (segment (start 152.4 104.14) (end 152.4 104.150974) (width 0.25) (layer "F.Cu") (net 13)))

